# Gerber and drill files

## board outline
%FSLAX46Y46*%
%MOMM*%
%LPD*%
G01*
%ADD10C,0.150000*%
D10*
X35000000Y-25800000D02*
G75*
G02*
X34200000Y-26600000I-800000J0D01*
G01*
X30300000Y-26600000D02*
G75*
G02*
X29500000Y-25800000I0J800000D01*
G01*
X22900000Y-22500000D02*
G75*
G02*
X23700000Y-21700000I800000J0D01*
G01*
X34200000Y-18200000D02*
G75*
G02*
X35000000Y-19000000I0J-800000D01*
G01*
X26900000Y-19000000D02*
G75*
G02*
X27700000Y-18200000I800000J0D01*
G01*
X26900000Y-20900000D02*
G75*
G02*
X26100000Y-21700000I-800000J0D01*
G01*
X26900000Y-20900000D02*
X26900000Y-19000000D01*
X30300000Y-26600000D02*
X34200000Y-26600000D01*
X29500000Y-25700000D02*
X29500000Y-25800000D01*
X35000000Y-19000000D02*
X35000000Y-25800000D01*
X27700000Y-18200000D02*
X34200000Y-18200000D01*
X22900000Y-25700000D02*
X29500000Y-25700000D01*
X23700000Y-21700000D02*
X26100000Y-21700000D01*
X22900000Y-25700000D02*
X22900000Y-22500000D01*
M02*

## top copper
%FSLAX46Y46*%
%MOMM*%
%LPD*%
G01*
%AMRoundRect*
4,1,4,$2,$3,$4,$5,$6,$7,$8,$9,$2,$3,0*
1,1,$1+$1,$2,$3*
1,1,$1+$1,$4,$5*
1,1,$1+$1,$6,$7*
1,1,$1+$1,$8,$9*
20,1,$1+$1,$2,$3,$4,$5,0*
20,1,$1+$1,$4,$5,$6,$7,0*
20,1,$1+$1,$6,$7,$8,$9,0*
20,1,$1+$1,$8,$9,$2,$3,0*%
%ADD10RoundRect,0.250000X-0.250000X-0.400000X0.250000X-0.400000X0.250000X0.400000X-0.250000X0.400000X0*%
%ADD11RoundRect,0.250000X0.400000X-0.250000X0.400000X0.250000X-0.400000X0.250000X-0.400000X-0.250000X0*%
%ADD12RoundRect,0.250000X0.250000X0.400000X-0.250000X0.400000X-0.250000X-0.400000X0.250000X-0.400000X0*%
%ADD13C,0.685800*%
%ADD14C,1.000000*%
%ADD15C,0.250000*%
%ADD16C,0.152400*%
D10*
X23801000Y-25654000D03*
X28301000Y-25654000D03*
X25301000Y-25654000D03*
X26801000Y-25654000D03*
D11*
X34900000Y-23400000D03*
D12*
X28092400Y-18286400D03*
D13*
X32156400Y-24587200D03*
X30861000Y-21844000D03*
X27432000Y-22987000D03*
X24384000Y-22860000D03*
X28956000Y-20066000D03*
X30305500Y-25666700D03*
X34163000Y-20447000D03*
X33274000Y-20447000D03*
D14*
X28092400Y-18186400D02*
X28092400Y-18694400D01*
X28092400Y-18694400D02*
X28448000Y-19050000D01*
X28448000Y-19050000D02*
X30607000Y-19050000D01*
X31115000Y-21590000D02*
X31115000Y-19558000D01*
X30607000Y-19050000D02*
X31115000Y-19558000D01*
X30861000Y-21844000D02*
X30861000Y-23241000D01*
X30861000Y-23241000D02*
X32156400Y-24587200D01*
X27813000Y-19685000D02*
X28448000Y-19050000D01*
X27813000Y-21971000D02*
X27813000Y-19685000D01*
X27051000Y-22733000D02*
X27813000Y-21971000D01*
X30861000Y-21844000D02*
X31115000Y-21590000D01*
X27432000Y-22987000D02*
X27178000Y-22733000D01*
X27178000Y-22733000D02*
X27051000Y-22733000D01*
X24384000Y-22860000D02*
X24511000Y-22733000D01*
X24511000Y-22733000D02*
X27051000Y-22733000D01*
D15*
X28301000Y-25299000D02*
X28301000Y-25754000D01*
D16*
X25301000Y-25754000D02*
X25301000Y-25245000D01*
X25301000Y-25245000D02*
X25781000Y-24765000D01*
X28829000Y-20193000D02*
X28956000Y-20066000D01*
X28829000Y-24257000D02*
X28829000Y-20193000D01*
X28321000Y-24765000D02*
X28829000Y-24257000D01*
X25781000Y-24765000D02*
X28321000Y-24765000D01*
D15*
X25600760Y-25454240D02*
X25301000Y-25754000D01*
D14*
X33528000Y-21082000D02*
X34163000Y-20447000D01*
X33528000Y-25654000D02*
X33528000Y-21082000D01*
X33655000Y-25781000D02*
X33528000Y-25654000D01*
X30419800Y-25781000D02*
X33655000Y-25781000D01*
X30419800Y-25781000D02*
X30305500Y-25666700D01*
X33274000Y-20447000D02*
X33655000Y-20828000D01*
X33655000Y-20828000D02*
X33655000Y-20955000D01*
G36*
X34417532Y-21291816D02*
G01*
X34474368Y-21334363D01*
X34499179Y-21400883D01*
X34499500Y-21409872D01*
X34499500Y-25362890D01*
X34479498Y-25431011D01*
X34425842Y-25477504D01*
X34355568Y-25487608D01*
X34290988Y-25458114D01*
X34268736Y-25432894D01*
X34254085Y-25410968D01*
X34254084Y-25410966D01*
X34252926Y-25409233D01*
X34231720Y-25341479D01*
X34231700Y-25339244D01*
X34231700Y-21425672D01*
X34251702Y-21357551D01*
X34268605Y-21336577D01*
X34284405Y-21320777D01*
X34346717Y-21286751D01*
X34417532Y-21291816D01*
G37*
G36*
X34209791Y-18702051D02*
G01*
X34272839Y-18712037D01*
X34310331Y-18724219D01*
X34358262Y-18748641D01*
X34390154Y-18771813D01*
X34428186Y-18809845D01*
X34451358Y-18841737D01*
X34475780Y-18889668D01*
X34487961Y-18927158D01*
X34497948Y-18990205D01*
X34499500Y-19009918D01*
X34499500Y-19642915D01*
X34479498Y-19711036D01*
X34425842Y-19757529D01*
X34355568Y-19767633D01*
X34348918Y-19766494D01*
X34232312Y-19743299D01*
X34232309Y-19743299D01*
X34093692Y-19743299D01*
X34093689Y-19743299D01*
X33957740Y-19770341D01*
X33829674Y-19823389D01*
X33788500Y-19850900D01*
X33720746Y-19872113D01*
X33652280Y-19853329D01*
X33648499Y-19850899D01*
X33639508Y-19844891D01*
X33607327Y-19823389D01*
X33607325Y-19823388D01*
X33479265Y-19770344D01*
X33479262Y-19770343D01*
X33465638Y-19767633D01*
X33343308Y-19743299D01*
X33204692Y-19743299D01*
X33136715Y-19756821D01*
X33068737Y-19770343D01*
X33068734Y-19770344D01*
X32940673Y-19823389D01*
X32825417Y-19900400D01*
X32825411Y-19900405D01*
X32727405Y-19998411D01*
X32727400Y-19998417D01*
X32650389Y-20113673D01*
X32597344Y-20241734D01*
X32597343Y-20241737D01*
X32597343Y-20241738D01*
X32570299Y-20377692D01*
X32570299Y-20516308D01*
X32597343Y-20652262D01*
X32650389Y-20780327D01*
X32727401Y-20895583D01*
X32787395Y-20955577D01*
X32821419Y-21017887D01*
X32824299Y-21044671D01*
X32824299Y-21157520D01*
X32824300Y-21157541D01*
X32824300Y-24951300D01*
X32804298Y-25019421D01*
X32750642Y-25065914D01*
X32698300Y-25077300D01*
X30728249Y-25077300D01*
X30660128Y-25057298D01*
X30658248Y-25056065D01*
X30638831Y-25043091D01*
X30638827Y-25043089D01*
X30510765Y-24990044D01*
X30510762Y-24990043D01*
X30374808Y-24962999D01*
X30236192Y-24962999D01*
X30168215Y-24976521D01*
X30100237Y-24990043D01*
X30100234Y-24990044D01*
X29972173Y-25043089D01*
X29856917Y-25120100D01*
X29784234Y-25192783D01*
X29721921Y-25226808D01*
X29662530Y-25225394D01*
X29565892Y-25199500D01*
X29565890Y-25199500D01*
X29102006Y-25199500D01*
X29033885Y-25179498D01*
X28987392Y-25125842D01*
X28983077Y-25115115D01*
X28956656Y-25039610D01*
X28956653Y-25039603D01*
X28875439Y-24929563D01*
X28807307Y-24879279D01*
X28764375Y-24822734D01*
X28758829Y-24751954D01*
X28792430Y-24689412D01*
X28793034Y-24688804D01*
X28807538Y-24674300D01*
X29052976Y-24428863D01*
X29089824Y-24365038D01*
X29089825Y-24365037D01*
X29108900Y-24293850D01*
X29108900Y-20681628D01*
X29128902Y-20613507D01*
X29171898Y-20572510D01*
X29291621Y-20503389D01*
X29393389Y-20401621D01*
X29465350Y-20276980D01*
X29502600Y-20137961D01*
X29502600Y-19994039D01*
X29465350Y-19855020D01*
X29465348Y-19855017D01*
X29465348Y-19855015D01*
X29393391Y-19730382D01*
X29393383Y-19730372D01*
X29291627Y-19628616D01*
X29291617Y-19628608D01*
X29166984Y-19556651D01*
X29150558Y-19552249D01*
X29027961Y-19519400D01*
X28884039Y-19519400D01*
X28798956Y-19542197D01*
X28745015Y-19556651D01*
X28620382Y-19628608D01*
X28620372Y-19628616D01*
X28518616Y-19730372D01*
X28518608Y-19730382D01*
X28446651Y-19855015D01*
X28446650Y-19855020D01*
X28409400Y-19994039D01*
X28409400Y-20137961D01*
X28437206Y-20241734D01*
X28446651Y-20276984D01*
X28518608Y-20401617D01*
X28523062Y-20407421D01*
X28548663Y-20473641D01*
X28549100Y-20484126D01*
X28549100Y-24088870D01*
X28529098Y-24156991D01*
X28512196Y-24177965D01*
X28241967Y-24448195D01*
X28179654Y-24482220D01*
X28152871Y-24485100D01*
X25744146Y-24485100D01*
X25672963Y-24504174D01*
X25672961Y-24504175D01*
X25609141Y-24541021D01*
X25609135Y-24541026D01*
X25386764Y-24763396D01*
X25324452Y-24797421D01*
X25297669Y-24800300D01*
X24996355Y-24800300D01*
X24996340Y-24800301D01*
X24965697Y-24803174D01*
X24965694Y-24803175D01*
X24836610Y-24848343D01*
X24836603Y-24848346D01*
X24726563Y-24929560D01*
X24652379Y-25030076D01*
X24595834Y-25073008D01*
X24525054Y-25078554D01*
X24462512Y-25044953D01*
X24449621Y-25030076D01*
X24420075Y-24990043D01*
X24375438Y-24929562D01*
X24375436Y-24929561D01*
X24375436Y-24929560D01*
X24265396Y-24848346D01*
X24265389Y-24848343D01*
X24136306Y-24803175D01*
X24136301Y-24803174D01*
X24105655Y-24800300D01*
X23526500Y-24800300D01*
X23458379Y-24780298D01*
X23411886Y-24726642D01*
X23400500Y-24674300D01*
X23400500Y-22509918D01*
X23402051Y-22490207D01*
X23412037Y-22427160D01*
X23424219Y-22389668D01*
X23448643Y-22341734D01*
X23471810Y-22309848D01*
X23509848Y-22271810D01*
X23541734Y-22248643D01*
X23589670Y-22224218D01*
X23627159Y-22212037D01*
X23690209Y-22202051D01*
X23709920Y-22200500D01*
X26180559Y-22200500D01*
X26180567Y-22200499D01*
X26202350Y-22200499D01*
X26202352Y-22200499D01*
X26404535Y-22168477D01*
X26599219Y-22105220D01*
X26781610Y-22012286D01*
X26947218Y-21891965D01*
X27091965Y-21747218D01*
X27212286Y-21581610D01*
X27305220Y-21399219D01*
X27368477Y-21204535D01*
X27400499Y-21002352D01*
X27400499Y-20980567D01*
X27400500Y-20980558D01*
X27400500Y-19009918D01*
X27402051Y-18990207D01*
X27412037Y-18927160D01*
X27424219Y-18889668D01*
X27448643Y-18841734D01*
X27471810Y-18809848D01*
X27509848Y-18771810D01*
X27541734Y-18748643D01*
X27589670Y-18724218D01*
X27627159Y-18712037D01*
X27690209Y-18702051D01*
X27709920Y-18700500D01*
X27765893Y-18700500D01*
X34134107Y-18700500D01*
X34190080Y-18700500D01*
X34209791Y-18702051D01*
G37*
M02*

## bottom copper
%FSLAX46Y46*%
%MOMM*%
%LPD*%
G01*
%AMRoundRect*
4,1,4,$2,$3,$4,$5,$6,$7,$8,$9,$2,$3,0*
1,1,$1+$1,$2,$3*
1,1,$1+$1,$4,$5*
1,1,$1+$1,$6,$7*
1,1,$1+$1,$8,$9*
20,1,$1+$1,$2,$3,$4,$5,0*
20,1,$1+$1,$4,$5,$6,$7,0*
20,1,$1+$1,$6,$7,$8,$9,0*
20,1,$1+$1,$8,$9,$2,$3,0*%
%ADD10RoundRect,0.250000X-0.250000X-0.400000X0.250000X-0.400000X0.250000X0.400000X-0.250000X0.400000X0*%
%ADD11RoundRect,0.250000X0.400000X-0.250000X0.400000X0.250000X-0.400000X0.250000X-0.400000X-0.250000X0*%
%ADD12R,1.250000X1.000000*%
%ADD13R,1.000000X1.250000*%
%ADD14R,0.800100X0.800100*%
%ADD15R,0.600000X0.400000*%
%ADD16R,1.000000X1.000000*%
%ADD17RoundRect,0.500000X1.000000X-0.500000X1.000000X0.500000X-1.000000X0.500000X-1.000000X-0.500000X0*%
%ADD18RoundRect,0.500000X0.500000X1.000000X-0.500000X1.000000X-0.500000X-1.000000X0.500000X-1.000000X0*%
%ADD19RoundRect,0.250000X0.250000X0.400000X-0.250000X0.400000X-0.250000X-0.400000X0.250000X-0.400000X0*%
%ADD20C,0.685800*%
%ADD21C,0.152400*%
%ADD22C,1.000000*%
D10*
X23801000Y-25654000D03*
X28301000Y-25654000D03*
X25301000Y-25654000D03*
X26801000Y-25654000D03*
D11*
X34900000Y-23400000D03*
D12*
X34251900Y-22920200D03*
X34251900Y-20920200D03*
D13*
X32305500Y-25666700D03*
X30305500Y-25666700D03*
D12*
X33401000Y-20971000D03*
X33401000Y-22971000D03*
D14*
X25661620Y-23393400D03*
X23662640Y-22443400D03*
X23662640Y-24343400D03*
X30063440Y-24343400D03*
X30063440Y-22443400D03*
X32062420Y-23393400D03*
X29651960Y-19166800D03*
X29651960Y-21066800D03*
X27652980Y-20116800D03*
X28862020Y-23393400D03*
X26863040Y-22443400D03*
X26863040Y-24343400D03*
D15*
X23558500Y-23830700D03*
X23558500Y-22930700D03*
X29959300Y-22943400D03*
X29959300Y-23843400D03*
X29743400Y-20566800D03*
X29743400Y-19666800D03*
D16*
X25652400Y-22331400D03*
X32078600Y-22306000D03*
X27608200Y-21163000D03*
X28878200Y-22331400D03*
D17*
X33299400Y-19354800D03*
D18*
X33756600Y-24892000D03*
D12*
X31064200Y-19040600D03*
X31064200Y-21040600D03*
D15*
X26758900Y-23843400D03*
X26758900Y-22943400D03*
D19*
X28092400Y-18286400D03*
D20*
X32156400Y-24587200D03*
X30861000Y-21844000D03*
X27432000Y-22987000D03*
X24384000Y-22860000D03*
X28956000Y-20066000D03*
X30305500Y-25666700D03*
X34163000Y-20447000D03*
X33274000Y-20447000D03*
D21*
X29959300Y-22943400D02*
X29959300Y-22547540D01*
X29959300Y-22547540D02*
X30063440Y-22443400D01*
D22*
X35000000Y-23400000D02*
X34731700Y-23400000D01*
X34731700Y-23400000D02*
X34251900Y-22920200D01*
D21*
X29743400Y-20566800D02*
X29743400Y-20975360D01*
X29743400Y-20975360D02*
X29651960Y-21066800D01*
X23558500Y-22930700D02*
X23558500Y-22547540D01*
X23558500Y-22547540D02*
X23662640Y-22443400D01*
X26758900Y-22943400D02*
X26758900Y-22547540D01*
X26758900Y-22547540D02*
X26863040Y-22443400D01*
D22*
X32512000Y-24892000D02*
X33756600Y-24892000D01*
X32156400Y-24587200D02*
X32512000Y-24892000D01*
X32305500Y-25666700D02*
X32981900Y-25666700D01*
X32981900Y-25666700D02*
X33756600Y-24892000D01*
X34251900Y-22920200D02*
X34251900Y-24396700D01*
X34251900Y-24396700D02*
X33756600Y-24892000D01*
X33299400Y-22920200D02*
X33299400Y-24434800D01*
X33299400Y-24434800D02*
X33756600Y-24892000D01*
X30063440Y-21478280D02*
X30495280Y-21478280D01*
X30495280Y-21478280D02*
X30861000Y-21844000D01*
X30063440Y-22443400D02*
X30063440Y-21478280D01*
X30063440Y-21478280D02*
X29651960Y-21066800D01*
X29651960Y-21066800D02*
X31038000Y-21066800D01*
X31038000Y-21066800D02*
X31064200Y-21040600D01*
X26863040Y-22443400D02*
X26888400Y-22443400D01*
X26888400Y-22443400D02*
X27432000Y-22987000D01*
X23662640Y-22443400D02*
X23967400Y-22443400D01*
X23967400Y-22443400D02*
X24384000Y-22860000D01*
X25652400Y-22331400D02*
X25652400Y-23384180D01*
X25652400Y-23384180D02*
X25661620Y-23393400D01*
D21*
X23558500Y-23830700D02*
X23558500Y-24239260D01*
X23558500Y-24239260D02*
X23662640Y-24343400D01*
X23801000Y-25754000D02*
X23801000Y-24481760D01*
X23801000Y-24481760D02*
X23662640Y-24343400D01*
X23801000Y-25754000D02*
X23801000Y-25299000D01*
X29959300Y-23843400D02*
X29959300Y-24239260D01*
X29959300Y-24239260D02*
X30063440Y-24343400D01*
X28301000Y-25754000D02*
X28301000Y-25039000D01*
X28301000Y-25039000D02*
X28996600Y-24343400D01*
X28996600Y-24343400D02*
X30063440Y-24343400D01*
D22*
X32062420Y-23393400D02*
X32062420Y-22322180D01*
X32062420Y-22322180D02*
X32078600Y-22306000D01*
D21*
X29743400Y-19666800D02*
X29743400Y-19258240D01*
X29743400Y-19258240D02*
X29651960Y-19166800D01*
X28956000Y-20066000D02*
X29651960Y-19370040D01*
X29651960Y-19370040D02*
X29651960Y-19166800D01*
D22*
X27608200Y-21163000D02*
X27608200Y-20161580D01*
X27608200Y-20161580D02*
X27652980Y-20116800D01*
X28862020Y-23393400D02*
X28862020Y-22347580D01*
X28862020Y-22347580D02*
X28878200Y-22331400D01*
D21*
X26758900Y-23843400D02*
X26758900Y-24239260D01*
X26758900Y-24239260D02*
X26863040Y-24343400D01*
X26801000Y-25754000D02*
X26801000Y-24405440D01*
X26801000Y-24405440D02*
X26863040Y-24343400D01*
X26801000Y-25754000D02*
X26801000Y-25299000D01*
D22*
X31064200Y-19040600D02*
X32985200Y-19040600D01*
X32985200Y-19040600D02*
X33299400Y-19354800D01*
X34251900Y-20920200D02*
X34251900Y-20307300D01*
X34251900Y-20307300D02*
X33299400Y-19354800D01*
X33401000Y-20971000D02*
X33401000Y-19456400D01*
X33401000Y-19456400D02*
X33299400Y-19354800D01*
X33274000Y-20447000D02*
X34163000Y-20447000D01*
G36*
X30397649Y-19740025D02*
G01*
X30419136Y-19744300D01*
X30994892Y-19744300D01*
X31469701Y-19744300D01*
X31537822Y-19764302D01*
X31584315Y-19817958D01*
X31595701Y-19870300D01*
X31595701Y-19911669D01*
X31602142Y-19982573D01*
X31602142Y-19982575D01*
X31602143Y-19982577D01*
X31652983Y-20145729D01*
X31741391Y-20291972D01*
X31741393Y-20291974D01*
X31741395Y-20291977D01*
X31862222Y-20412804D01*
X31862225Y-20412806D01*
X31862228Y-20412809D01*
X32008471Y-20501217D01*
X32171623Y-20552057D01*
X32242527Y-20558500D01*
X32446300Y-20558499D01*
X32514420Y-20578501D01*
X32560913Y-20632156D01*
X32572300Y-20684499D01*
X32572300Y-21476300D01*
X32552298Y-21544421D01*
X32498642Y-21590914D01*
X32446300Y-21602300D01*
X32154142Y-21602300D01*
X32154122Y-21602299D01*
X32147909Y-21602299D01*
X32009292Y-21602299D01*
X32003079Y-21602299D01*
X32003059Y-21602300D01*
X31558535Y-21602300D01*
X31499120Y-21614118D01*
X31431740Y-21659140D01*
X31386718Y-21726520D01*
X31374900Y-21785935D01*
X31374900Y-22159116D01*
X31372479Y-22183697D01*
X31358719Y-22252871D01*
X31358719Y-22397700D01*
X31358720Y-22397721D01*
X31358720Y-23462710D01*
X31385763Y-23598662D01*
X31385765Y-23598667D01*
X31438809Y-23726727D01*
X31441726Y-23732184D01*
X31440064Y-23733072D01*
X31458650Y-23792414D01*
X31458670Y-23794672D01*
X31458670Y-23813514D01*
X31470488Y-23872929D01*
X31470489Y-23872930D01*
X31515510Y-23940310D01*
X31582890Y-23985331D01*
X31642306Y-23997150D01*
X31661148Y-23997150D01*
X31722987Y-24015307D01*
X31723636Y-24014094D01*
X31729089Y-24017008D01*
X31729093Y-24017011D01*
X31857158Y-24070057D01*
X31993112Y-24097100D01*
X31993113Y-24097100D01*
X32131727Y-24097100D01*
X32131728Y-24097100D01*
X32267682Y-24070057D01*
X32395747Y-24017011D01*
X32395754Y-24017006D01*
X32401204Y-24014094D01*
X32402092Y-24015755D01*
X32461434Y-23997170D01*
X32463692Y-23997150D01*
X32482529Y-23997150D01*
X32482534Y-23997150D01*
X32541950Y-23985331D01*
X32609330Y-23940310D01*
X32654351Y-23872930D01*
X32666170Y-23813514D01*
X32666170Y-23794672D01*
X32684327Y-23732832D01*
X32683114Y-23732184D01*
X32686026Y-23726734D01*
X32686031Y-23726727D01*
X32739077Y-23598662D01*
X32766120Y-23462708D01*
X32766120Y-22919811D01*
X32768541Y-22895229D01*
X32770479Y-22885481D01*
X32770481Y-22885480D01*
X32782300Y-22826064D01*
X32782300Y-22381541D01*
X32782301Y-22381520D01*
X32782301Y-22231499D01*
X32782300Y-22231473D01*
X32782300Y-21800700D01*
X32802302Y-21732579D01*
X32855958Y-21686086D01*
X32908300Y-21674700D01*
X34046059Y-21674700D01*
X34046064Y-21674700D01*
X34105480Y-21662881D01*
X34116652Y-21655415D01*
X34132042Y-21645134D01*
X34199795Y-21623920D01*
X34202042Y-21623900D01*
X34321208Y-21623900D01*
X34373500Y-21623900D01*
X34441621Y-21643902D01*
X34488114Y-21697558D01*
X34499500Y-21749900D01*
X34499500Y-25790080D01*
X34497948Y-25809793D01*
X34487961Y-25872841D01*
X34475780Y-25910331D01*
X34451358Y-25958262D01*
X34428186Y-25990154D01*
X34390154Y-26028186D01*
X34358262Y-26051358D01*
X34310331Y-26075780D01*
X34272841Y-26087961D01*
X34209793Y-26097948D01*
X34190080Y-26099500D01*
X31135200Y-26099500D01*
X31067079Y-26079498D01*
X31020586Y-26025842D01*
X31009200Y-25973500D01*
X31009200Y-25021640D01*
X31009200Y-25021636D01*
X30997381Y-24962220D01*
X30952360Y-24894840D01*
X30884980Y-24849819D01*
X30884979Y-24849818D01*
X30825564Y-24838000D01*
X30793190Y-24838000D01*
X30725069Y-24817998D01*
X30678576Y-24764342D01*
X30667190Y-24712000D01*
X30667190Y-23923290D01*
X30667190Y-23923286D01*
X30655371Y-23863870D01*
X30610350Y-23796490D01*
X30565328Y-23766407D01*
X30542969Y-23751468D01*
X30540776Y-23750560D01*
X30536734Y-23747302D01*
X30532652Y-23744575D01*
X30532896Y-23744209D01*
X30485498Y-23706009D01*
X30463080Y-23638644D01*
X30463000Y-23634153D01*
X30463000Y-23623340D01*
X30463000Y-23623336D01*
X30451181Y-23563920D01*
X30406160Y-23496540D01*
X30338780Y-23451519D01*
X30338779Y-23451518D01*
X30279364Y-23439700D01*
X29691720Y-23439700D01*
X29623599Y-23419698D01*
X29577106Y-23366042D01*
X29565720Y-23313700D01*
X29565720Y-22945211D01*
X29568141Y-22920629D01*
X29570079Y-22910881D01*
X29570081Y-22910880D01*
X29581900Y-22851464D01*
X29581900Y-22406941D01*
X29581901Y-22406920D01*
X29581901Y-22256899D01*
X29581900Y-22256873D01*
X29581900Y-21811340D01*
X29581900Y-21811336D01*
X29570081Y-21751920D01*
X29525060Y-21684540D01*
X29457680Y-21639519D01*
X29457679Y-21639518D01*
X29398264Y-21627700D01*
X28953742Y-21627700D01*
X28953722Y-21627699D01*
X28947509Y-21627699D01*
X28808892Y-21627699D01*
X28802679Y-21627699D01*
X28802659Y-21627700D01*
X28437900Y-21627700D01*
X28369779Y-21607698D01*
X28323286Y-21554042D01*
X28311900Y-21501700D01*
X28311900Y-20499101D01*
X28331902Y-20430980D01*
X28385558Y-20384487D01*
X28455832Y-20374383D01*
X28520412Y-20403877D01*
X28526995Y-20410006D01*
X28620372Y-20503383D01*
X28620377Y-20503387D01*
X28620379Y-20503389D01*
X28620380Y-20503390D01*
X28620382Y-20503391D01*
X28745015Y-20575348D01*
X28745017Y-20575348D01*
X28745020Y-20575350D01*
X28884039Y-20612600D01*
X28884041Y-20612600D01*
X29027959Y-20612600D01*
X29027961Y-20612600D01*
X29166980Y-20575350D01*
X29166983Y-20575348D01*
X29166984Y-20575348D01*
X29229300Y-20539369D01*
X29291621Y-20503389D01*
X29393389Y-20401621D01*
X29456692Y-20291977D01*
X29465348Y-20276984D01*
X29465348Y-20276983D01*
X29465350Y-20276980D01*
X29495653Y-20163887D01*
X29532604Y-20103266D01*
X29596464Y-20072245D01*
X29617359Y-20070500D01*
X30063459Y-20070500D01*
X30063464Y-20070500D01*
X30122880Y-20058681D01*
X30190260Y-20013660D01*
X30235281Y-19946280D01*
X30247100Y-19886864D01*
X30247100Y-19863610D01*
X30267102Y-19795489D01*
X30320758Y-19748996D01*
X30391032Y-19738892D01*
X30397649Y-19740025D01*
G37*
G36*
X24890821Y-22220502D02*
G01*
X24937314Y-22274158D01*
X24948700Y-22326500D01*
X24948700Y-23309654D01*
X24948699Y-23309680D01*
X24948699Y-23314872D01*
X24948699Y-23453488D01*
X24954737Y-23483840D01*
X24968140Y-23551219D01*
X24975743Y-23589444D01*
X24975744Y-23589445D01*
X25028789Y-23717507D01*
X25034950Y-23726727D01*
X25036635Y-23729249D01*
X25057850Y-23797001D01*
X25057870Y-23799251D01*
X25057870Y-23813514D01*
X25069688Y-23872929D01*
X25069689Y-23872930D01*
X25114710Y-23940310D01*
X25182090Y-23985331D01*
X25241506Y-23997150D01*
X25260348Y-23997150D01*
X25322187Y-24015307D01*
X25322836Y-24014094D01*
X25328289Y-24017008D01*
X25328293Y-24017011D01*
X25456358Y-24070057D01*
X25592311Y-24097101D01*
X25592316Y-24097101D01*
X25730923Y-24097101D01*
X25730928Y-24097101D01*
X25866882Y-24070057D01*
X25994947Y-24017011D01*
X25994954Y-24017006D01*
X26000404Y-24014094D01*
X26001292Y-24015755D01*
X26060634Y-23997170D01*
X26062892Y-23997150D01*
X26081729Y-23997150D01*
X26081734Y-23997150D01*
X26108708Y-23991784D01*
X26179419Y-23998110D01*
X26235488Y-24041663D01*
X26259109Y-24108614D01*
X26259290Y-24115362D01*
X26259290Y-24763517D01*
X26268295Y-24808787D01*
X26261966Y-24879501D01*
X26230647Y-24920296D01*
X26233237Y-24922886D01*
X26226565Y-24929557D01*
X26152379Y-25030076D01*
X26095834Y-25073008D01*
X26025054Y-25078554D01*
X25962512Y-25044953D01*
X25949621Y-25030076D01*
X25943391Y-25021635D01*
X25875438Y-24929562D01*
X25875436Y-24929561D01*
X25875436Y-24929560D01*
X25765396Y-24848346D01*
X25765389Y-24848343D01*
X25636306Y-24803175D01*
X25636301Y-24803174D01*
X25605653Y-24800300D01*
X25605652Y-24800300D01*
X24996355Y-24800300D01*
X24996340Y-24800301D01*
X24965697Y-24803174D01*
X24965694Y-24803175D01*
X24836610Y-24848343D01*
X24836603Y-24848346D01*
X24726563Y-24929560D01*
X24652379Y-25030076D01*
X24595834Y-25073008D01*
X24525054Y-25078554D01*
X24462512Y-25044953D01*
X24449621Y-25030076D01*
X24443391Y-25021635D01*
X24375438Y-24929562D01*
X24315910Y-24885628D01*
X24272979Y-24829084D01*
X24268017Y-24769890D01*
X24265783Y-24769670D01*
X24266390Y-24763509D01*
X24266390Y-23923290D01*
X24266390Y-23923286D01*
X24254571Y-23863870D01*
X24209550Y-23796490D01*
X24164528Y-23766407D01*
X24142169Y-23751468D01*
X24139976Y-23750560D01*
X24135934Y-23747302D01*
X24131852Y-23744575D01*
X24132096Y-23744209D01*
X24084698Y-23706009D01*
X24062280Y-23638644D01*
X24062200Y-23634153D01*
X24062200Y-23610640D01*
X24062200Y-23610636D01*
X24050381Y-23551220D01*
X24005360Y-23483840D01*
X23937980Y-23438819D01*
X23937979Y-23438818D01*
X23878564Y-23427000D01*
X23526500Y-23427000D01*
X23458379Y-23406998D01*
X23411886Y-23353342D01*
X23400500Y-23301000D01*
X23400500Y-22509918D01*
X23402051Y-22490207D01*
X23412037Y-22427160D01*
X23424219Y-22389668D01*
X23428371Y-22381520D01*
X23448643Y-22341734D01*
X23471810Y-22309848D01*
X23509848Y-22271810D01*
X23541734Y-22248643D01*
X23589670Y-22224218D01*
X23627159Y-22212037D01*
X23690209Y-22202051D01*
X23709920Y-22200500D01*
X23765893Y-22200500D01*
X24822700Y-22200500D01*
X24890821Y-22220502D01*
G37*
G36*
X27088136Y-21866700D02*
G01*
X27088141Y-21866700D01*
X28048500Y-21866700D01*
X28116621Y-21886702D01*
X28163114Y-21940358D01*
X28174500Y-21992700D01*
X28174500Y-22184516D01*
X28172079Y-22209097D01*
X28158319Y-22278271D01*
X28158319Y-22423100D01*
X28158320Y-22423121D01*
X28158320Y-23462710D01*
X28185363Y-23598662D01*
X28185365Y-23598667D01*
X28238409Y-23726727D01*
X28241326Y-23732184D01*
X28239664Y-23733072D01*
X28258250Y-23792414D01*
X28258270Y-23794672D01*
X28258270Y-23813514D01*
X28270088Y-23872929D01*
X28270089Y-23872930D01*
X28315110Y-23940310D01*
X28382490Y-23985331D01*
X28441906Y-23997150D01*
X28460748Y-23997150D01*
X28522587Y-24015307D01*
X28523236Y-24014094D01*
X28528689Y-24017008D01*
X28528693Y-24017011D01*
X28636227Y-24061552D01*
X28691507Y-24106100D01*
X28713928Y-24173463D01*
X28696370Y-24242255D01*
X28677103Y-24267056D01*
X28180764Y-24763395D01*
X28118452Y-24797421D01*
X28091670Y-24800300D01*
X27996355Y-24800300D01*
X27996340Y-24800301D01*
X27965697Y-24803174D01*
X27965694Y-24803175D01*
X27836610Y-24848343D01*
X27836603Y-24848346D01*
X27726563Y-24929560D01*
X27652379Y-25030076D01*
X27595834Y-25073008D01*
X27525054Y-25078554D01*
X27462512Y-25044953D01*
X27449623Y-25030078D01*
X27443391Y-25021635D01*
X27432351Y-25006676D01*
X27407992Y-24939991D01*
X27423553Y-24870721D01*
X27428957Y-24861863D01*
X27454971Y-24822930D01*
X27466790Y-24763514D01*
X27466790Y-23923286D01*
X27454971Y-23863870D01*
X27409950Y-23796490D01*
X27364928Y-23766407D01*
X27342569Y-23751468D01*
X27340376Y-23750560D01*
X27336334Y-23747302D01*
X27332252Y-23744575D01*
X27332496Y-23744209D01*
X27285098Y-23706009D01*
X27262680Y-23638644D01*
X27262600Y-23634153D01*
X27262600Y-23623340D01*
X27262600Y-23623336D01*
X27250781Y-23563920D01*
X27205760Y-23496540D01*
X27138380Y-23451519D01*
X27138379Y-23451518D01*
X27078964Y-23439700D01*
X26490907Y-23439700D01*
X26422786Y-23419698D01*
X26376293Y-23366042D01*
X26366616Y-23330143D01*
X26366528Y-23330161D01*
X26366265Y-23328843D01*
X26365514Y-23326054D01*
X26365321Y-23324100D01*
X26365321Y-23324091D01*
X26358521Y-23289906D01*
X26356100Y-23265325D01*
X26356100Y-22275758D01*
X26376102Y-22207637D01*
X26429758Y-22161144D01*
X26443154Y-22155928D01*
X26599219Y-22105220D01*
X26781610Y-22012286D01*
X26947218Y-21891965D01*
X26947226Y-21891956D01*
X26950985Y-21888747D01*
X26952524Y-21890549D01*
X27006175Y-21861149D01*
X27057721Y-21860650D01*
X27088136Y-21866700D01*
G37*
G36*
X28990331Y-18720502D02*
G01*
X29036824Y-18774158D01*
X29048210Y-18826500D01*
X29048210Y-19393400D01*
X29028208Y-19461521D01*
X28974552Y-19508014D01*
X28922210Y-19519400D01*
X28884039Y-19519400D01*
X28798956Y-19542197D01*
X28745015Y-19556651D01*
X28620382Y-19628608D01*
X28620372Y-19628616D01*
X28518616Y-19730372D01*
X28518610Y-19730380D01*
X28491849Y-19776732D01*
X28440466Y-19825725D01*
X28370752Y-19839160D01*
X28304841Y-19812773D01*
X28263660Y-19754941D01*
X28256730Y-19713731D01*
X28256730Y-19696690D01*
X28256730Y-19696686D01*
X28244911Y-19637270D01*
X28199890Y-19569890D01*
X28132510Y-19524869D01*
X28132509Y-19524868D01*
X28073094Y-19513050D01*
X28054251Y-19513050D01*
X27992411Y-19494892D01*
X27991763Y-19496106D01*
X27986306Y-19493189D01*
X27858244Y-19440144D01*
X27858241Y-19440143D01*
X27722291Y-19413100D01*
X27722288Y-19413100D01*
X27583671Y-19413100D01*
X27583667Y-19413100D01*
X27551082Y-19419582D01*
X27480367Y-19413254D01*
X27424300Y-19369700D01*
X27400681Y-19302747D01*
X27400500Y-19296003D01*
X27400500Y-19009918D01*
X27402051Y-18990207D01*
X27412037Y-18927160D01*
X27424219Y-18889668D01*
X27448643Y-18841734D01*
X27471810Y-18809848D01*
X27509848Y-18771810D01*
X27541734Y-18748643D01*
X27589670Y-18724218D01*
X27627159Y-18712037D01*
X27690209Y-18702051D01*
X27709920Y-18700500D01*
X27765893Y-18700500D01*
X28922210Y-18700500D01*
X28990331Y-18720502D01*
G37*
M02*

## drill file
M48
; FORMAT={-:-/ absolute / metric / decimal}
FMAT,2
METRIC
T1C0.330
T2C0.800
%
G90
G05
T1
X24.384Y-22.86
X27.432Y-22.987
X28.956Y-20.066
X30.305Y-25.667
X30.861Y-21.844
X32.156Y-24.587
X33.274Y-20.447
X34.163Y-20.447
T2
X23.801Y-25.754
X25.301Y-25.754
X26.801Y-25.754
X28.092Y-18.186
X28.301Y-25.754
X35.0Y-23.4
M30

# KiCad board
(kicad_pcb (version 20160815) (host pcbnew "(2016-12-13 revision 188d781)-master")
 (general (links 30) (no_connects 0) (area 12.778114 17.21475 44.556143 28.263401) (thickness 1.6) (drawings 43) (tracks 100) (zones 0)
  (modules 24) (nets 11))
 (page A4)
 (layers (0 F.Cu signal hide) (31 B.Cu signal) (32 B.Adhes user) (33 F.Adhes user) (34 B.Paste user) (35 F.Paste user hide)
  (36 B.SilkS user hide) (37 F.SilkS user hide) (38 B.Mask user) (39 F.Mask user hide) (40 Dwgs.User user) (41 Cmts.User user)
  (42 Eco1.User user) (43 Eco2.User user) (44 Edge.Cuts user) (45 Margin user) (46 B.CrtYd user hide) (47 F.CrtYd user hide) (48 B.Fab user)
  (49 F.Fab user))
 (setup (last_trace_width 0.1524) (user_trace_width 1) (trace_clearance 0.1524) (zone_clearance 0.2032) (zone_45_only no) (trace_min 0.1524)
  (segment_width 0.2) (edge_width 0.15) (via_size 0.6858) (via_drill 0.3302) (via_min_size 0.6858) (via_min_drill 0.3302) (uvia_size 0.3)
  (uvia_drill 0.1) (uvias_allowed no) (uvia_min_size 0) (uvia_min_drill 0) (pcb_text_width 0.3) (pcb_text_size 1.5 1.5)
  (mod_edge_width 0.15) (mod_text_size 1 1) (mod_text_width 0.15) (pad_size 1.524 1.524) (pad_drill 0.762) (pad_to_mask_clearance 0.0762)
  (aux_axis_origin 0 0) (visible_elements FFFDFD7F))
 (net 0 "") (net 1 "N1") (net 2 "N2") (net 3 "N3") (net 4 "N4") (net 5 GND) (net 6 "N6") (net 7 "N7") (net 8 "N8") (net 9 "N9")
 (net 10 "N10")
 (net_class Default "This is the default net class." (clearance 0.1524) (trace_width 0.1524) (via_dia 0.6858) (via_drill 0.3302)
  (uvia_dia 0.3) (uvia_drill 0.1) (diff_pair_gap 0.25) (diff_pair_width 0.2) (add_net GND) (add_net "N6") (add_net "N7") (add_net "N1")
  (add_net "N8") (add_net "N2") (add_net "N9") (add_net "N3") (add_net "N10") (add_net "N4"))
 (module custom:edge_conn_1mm (layer F.Cu) (at 23.801 25.754)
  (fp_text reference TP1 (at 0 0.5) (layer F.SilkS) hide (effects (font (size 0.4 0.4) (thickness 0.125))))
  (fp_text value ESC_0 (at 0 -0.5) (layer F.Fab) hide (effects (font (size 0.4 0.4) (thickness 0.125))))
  (pad 1 thru_hole roundrect (at 0 0) (size 1 1.3) (drill 0.8 (offset 0 -0.1)) (layers *.Cu *.Mask) (roundrect_rratio 0.25) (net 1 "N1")))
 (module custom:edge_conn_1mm (layer F.Cu) (at 28.301 25.754)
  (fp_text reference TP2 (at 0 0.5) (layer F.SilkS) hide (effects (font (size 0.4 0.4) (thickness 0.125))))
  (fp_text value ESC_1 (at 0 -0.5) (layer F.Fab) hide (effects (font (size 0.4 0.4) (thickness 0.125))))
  (pad 1 thru_hole roundrect (at 0 0) (size 1 1.3) (drill 0.8 (offset 0 -0.1)) (layers *.Cu *.Mask) (roundrect_rratio 0.25) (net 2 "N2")))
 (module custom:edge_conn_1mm (layer F.Cu) (at 25.301 25.754)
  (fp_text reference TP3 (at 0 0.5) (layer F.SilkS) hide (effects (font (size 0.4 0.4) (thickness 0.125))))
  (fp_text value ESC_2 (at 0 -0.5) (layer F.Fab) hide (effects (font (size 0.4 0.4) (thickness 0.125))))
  (pad 1 thru_hole roundrect (at 0 0) (size 1 1.3) (drill 0.8 (offset 0 -0.1)) (layers *.Cu *.Mask) (roundrect_rratio 0.25) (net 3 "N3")))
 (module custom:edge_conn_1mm (layer F.Cu) (at 26.801 25.754)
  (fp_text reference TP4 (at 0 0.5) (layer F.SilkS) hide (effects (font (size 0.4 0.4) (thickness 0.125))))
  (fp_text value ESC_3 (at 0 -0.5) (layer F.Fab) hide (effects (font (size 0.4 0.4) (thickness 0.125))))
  (pad 1 thru_hole roundrect (at 0 0) (size 1 1.3) (drill 0.8 (offset 0 -0.1)) (layers *.Cu *.Mask) (roundrect_rratio 0.25) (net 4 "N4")))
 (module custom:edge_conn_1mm (layer F.Cu) (at 35 23.4 90)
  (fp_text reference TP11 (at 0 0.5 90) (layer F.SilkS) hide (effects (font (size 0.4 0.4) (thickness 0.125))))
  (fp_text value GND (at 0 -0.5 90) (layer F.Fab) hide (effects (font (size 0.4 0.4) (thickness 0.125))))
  (pad 1 thru_hole roundrect (at 0 0 90) (size 1 1.3) (drill 0.8 (offset 0 -0.1)) (layers *.Cu *.Mask) (roundrect_rratio 0.25) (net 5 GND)))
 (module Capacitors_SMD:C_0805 (layer B.Cu) (at 34.2519 21.9202 270)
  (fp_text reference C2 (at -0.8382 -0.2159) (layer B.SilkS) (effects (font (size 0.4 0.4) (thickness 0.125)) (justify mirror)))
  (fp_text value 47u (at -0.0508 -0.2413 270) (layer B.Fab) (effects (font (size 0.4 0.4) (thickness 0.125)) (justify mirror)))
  (pad 2 smd rect (at 1 0 270) (size 1 1.25) (layers B.Cu B.Paste B.Mask) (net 5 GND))
  (pad 1 smd rect (at -1 0 270) (size 1 1.25) (layers B.Cu B.Paste B.Mask) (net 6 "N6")))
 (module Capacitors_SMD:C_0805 (layer B.Cu) (at 31.3055 25.6667)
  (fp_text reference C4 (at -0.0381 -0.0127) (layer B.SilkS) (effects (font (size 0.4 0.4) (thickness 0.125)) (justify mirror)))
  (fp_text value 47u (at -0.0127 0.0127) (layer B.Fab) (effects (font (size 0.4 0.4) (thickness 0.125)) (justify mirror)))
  (pad 2 smd rect (at 1 0) (size 1 1.25) (layers B.Cu B.Paste B.Mask) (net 5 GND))
  (pad 1 smd rect (at -1 0) (size 1 1.25) (layers B.Cu B.Paste B.Mask) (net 6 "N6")))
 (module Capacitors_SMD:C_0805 (layer B.Cu) (at 33.401 21.971 270)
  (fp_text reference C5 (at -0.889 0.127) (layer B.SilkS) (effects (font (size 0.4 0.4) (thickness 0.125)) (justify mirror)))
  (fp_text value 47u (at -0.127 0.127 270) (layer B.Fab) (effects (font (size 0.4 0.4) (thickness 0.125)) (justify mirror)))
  (pad 1 smd rect (at -1 0 270) (size 1 1.25) (layers B.Cu B.Paste B.Mask) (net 6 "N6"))
  (pad 2 smd rect (at 1 0 270) (size 1 1.25) (layers B.Cu B.Paste B.Mask) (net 5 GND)))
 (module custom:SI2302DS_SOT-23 (layer B.Cu) (at 24.6634 23.3934 90)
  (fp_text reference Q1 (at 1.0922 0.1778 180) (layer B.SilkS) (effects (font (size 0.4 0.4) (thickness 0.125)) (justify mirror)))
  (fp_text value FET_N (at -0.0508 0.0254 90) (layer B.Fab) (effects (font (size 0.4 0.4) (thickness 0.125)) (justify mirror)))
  (pad D smd rect (at 0 0.99822 90) (size 0.8001 0.8001) (layers B.Cu B.Paste B.Mask) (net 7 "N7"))
  (pad S smd rect (at 0.95 -1.00076 90) (size 0.8001 0.8001) (layers B.Cu B.Paste B.Mask) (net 5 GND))
  (pad G smd rect (at -0.95 -1.00076 90) (size 0.8001 0.8001) (layers B.Cu B.Paste B.Mask) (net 1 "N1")))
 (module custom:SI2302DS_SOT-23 (layer B.Cu) (at 31.0642 23.3934 90)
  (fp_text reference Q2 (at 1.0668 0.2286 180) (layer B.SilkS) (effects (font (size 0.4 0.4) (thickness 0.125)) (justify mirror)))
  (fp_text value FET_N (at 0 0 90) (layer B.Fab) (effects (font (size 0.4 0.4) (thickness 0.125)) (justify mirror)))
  (pad G smd rect (at -0.95 -1.00076 90) (size 0.8001 0.8001) (layers B.Cu B.Paste B.Mask) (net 2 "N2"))
  (pad S smd rect (at 0.95 -1.00076 90) (size 0.8001 0.8001) (layers B.Cu B.Paste B.Mask) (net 5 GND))
  (pad D smd rect (at 0 0.99822 90) (size 0.8001 0.8001) (layers B.Cu B.Paste B.Mask) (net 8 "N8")))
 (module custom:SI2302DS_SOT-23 (layer B.Cu) (at 28.6512 20.1168 270)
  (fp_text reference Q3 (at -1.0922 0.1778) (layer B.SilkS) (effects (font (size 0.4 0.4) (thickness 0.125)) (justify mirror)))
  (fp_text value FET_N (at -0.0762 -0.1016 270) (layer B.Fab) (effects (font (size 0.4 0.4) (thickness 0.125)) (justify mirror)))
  (pad G smd rect (at -0.95 -1.00076 270) (size 0.8001 0.8001) (layers B.Cu B.Paste B.Mask) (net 3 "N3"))
  (pad S smd rect (at 0.95 -1.00076 270) (size 0.8001 0.8001) (layers B.Cu B.Paste B.Mask) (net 5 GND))
  (pad D smd rect (at 0 0.99822 270) (size 0.8001 0.8001) (layers B.Cu B.Paste B.Mask) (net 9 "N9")))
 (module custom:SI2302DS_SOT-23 (layer B.Cu) (at 27.8638 23.3934 90)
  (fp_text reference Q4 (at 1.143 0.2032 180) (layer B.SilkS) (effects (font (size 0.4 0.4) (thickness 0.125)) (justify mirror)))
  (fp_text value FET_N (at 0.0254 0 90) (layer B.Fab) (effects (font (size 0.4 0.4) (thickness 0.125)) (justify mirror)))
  (pad D smd rect (at 0 0.99822 90) (size 0.8001 0.8001) (layers B.Cu B.Paste B.Mask) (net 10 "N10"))
  (pad S smd rect (at 0.95 -1.00076 90) (size 0.8001 0.8001) (layers B.Cu B.Paste B.Mask) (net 5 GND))
  (pad G smd rect (at -0.95 -1.00076 90) (size 0.8001 0.8001) (layers B.Cu B.Paste B.Mask) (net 4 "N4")))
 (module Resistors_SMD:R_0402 (layer B.Cu) (at 23.5585 23.3807 90)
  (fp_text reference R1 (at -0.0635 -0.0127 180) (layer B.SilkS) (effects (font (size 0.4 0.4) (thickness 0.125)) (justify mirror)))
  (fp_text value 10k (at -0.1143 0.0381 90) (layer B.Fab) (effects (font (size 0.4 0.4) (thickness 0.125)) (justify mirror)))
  (pad 1 smd rect (at -0.45 0 90) (size 0.4 0.6) (layers B.Cu B.Paste B.Mask) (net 1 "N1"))
  (pad 2 smd rect (at 0.45 0 90) (size 0.4 0.6) (layers B.Cu B.Paste B.Mask) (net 5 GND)))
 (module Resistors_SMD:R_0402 (layer B.Cu) (at 29.9593 23.3934 90)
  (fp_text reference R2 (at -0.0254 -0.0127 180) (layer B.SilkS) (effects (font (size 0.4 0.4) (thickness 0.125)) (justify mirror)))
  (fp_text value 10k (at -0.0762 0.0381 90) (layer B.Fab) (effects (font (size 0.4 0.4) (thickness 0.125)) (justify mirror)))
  (pad 2 smd rect (at 0.45 0 90) (size 0.4 0.6) (layers B.Cu B.Paste B.Mask) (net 5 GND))
  (pad 1 smd rect (at -0.45 0 90) (size 0.4 0.6) (layers B.Cu B.Paste B.Mask) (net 2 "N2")))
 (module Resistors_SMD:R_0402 (layer B.Cu) (at 29.7434 20.1168 270)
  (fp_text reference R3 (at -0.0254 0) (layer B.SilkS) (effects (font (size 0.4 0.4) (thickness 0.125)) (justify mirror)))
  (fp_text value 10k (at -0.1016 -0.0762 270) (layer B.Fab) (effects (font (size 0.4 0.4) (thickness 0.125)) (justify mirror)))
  (pad 2 smd rect (at 0.45 0 270) (size 0.4 0.6) (layers B.Cu B.Paste B.Mask) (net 5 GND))
  (pad 1 smd rect (at -0.45 0 270) (size 0.4 0.6) (layers B.Cu B.Paste B.Mask) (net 3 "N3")))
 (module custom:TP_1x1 (layer B.Cu) (at 25.5524 22.6314)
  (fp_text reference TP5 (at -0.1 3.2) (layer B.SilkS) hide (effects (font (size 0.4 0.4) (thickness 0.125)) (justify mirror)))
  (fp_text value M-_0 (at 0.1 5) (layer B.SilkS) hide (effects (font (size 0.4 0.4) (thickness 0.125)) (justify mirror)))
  (pad 1 smd rect (at 0.1 -0.3) (size 1 1) (layers B.Cu B.Mask) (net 7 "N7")))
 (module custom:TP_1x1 (layer B.Cu) (at 31.9786 22.606)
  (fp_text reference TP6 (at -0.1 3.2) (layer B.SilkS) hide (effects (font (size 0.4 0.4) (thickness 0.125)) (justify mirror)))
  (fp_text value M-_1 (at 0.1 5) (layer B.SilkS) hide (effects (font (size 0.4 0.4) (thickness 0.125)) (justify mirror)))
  (pad 1 smd rect (at 0.1 -0.3) (size 1 1) (layers B.Cu B.Mask) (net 8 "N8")))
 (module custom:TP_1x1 (layer B.Cu) (at 27.5082 21.463)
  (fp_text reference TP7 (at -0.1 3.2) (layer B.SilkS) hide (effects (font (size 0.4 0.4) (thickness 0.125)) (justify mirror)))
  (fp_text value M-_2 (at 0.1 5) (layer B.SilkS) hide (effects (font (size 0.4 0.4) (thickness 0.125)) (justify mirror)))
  (pad 1 smd rect (at 0.1 -0.3) (size 1 1) (layers B.Cu B.Mask) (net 9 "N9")))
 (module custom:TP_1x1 (layer B.Cu) (at 28.7782 22.6314)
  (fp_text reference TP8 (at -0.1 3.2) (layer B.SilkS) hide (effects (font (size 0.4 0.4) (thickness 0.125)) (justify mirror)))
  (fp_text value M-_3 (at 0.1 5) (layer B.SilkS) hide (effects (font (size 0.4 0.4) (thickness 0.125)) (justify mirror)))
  (pad 1 smd rect (at 0.1 -0.3) (size 1 1) (layers B.Cu B.Mask) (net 10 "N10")))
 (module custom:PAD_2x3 (layer B.Cu) (at 33.2994 19.3548 90)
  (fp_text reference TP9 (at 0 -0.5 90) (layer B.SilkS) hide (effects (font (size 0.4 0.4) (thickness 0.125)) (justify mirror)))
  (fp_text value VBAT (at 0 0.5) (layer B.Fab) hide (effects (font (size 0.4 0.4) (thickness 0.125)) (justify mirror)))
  (pad 1 smd roundrect (at 0 0 90) (size 2 3) (layers B.Cu B.Mask) (roundrect_rratio 0.25) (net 6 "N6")))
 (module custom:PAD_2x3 (layer B.Cu) (at 33.7566 24.892 180)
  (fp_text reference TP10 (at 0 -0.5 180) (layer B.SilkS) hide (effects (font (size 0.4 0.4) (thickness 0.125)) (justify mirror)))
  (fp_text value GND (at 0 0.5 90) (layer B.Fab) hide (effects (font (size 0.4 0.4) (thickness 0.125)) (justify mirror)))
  (pad 1 smd roundrect (at 0 0 180) (size 2 3) (layers B.Cu B.Mask) (roundrect_rratio 0.25) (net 5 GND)))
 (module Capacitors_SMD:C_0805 (layer B.Cu) (at 31.0642 20.0406 270)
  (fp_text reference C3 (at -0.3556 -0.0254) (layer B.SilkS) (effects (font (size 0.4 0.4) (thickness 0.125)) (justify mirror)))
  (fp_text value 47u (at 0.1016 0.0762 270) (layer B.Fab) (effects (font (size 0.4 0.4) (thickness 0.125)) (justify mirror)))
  (pad 1 smd rect (at -1 0 270) (size 1 1.25) (layers B.Cu B.Paste B.Mask) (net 6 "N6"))
  (pad 2 smd rect (at 1 0 270) (size 1 1.25) (layers B.Cu B.Paste B.Mask) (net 5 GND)))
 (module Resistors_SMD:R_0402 (layer B.Cu) (at 26.7589 23.3934 90)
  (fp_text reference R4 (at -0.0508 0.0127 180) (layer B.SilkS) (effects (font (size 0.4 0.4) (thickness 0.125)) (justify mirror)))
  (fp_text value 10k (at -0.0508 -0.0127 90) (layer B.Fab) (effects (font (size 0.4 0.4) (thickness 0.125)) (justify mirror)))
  (pad 1 smd rect (at -0.45 0 90) (size 0.4 0.6) (layers B.Cu B.Paste B.Mask) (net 4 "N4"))
  (pad 2 smd rect (at 0.45 0 90) (size 0.4 0.6) (layers B.Cu B.Paste B.Mask) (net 5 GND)))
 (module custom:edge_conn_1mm (layer F.Cu) (at 28.0924 18.1864 180)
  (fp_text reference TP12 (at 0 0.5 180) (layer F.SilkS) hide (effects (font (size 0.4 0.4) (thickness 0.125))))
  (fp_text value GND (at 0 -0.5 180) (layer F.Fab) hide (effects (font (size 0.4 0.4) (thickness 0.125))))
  (pad 1 thru_hole roundrect (at 0 0 180) (size 1 1.3) (drill 0.8 (offset 0 -0.1)) (layers *.Cu *.Mask) (roundrect_rratio 0.25) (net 5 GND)))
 (gr_arc (start 34.2 25.8) (end 35 25.8) (angle 90) (layer Edge.Cuts) (width 0.15))
 (gr_arc (start 30.3 25.8) (end 30.3 26.6) (angle 90) (layer Edge.Cuts) (width 0.15))
 (gr_arc (start 23.7 22.5) (end 22.9 22.5) (angle 90) (layer Edge.Cuts) (width 0.15))
 (gr_arc (start 34.2 19) (end 34.2 18.2) (angle 90) (layer Edge.Cuts) (width 0.15))
 (gr_arc (start 27.7 19) (end 26.9 19) (angle 90) (layer Edge.Cuts) (width 0.15))
 (gr_arc (start 26.1 20.9) (end 26.9 20.9) (angle 90) (layer Edge.Cuts) (width 0.15))
 (gr_line (start 26.9 20.9) (end 26.9 19) (angle 90) (layer Edge.Cuts) (width 0.15))
 (gr_line (start 30.3 26.6) (end 34.2 26.6) (angle 90) (layer Edge.Cuts) (width 0.15))
 (gr_line (start 29.5 25.7) (end 29.5 25.8) (angle 90) (layer Edge.Cuts) (width 0.15))
 (gr_line (start 35 19) (end 35 25.8) (angle 90) (layer Edge.Cuts) (width 0.15))
 (gr_line (start 27.7 18.2) (end 34.2 18.2) (angle 90) (layer Edge.Cuts) (width 0.15))
 (gr_line (start 22.9 25.7) (end 29.5 25.7) (angle 90) (layer Edge.Cuts) (width 0.15))
 (gr_line (start 23.7 21.7) (end 26.1 21.7) (angle 90) (layer Edge.Cuts) (width 0.15))
 (gr_line (start 22.9 25.7) (end 22.9 22.5) (angle 90) (layer Edge.Cuts) (width 0.15))
 (segment (start 28.0924 18.1864) (end 28.0924 18.6944) (width 1) (layer F.Cu) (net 5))
 (segment (start 28.0924 18.6944) (end 28.448 19.05) (width 1) (layer F.Cu) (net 5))
 (segment (start 29.9593 22.9434) (end 29.9593 22.54754) (width 0.1524) (layer B.Cu) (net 5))
 (segment (start 29.9593 22.54754) (end 30.06344 22.4434) (width 0.1524) (layer B.Cu) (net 5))
 (segment (start 35 23.4) (end 34.7317 23.4) (width 1) (layer B.Cu) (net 5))
 (segment (start 34.7317 23.4) (end 34.2519 22.9202) (width 1) (layer B.Cu) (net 5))
 (segment (start 28.448 19.05) (end 30.607 19.05) (width 1) (layer F.Cu) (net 5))
 (segment (start 31.115 21.59) (end 31.115 19.558) (width 1) (layer F.Cu) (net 5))
 (segment (start 30.607 19.05) (end 31.115 19.558) (width 1) (layer F.Cu) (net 5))
 (segment (start 29.7434 20.5668) (end 29.7434 20.97536) (width 0.1524) (layer B.Cu) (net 5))
 (segment (start 29.7434 20.97536) (end 29.65196 21.0668) (width 0.1524) (layer B.Cu) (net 5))
 (segment (start 23.5585 22.9307) (end 23.5585 22.54754) (width 0.1524) (layer B.Cu) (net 5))
 (segment (start 23.5585 22.54754) (end 23.66264 22.4434) (width 0.1524) (layer B.Cu) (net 5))
 (segment (start 26.7589 22.9434) (end 26.7589 22.54754) (width 0.1524) (layer B.Cu) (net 5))
 (segment (start 26.7589 22.54754) (end 26.86304 22.4434) (width 0.1524) (layer B.Cu) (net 5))
 (segment (start 30.861 21.844) (end 30.861 23.241) (width 1) (layer F.Cu) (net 5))
 (segment (start 32.512 24.892) (end 33.7566 24.892) (width 1) (layer B.Cu) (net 5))
 (segment (start 32.1564 24.5872) (end 32.512 24.892) (width 1) (layer B.Cu) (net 5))
 (via (at 32.1564 24.5872) (size 0.6858) (drill 0.3302) (layers F.Cu B.Cu) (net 5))
 (segment (start 30.861 23.241) (end 32.1564 24.5872) (width 1) (layer F.Cu) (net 5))
 (segment (start 32.3055 25.6667) (end 32.9819 25.6667) (width 1) (layer B.Cu) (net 5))
 (segment (start 32.9819 25.6667) (end 33.7566 24.892) (width 1) (layer B.Cu) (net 5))
 (segment (start 34.2519 22.9202) (end 34.2519 24.3967) (width 1) (layer B.Cu) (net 5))
 (segment (start 34.2519 24.3967) (end 33.7566 24.892) (width 1) (layer B.Cu) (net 5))
 (segment (start 33.2994 22.9202) (end 33.2994 24.4348) (width 1) (layer B.Cu) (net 5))
 (segment (start 33.2994 24.4348) (end 33.7566 24.892) (width 1) (layer B.Cu) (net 5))
 (segment (start 30.06344 21.47828) (end 30.49528 21.47828) (width 1) (layer B.Cu) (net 5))
 (segment (start 30.49528 21.47828) (end 30.861 21.844) (width 1) (layer B.Cu) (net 5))
 (segment (start 27.813 19.685) (end 28.448 19.05) (width 1) (layer F.Cu) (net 5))
 (segment (start 27.813 21.971) (end 27.813 19.685) (width 1) (layer F.Cu) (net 5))
 (segment (start 27.051 22.733) (end 27.813 21.971) (width 1) (layer F.Cu) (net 5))
 (segment (start 30.861 21.844) (end 31.115 21.59) (width 1) (layer F.Cu) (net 5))
 (via (at 30.861 21.844) (size 0.6858) (drill 0.3302) (layers F.Cu B.Cu) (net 5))
 (segment (start 30.06344 22.4434) (end 30.06344 21.47828) (width 1) (layer B.Cu) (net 5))
 (segment (start 30.06344 21.47828) (end 29.65196 21.0668) (width 1) (layer B.Cu) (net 5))
 (segment (start 29.65196 21.0668) (end 31.038 21.0668) (width 1) (layer B.Cu) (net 5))
 (segment (start 31.038 21.0668) (end 31.0642 21.0406) (width 1) (layer B.Cu) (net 5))
 (segment (start 26.86304 22.4434) (end 26.8884 22.4434) (width 1) (layer B.Cu) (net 5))
 (segment (start 26.8884 22.4434) (end 27.432 22.987) (width 1) (layer B.Cu) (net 5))
 (via (at 27.432 22.987) (size 0.6858) (drill 0.3302) (layers F.Cu B.Cu) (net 5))
 (segment (start 27.432 22.987) (end 27.178 22.733) (width 1) (layer F.Cu) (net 5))
 (segment (start 27.178 22.733) (end 27.051 22.733) (width 1) (layer F.Cu) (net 5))
 (segment (start 23.66264 22.4434) (end 23.9674 22.4434) (width 1) (layer B.Cu) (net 5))
 (segment (start 23.9674 22.4434) (end 24.384 22.86) (width 1) (layer B.Cu) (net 5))
 (via (at 24.384 22.86) (size 0.6858) (drill 0.3302) (layers F.Cu B.Cu) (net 5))
 (segment (start 24.384 22.86) (end 24.511 22.733) (width 1) (layer F.Cu) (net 5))
 (segment (start 24.511 22.733) (end 27.051 22.733) (width 1) (layer F.Cu) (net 5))
 (segment (start 25.6524 22.3314) (end 25.6524 23.38418) (width 1) (layer B.Cu) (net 7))
 (segment (start 25.6524 23.38418) (end 25.66162 23.3934) (width 1) (layer B.Cu) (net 7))
 (segment (start 23.5585 23.8307) (end 23.5585 24.23926) (width 0.1524) (layer B.Cu) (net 1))
 (segment (start 23.5585 24.23926) (end 23.66264 24.3434) (width 0.1524) (layer B.Cu) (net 1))
 (segment (start 23.801 25.754) (end 23.801 24.48176) (width 0.1524) (layer B.Cu) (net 1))
 (segment (start 23.801 24.48176) (end 23.66264 24.3434) (width 0.1524) (layer B.Cu) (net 1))
 (segment (start 23.801 25.754) (end 23.801 25.299) (width 0.1524) (layer B.Cu) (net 1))
 (segment (start 29.9593 23.8434) (end 29.9593 24.23926) (width 0.1524) (layer B.Cu) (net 2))
 (segment (start 29.9593 24.23926) (end 30.06344 24.3434) (width 0.1524) (layer B.Cu) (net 2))
 (segment (start 28.301 25.754) (end 28.301 25.039) (width 0.1524) (layer B.Cu) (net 2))
 (segment (start 28.301 25.039) (end 28.9966 24.3434) (width 0.1524) (layer B.Cu) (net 2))
 (segment (start 28.9966 24.3434) (end 30.06344 24.3434) (width 0.1524) (layer B.Cu) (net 2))
 (segment (start 28.301 25.299) (end 28.301 25.754) (width 0.25) (layer F.Cu) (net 2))
 (segment (start 32.06242 23.3934) (end 32.06242 22.32218) (width 1) (layer B.Cu) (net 8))
 (segment (start 32.06242 22.32218) (end 32.0786 22.306) (width 1) (layer B.Cu) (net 8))
 (segment (start 29.7434 19.6668) (end 29.7434 19.25824) (width 0.1524) (layer B.Cu) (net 3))
 (segment (start 29.7434 19.25824) (end 29.65196 19.1668) (width 0.1524) (layer B.Cu) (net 3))
 (segment (start 25.301 25.754) (end 25.301 25.245) (width 0.1524) (layer F.Cu) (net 3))
 (segment (start 25.301 25.245) (end 25.781 24.765) (width 0.1524) (layer F.Cu) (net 3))
 (segment (start 28.956 20.066) (end 29.65196 19.37004) (width 0.1524) (layer B.Cu) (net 3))
 (via (at 28.956 20.066) (size 0.6858) (drill 0.3302) (layers F.Cu B.Cu) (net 3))
 (segment (start 28.829 20.193) (end 28.956 20.066) (width 0.1524) (layer F.Cu) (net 3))
 (segment (start 28.829 24.257) (end 28.829 20.193) (width 0.1524) (layer F.Cu) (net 3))
 (segment (start 28.321 24.765) (end 28.829 24.257) (width 0.1524) (layer F.Cu) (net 3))
 (segment (start 25.781 24.765) (end 28.321 24.765) (width 0.1524) (layer F.Cu) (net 3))
 (segment (start 29.65196 19.37004) (end 29.65196 19.1668) (width 0.1524) (layer B.Cu) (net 3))
 (segment (start 25.60076 25.45424) (end 25.301 25.754) (width 0.25) (layer F.Cu) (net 3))
 (segment (start 27.6082 21.163) (end 27.6082 20.16158) (width 1) (layer B.Cu) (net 9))
 (segment (start 27.6082 20.16158) (end 27.65298 20.1168) (width 1) (layer B.Cu) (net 9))
 (segment (start 28.86202 23.3934) (end 28.86202 22.34758) (width 1) (layer B.Cu) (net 10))
 (segment (start 28.86202 22.34758) (end 28.8782 22.3314) (width 1) (layer B.Cu) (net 10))
 (segment (start 26.7589 23.8434) (end 26.7589 24.23926) (width 0.1524) (layer B.Cu) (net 4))
 (segment (start 26.7589 24.23926) (end 26.86304 24.3434) (width 0.1524) (layer B.Cu) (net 4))
 (segment (start 26.801 25.754) (end 26.801 24.40544) (width 0.1524) (layer B.Cu) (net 4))
 (segment (start 26.801 24.40544) (end 26.86304 24.3434) (width 0.1524) (layer B.Cu) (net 4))
 (segment (start 26.801 25.754) (end 26.801 25.299) (width 0.1524) (layer B.Cu) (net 4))
 (segment (start 31.0642 19.0406) (end 32.9852 19.0406) (width 1) (layer B.Cu) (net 6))
 (segment (start 32.9852 19.0406) (end 33.2994 19.3548) (width 1) (layer B.Cu) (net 6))
 (segment (start 34.2519 20.9202) (end 34.2519 20.3073) (width 1) (layer B.Cu) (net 6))
 (segment (start 34.2519 20.3073) (end 33.2994 19.3548) (width 1) (layer B.Cu) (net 6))
 (segment (start 33.401 20.971) (end 33.401 19.4564) (width 1) (layer B.Cu) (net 6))
 (segment (start 33.401 19.4564) (end 33.2994 19.3548) (width 1) (layer B.Cu) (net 6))
 (via (at 30.3055 25.6667) (size 0.6858) (drill 0.3302) (layers F.Cu B.Cu) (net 6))
 (segment (start 33.274 20.447) (end 34.163 20.447) (width 1) (layer B.Cu) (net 6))
 (via (at 34.163 20.447) (size 0.6858) (drill 0.3302) (layers F.Cu B.Cu) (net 6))
 (segment (start 33.528 21.082) (end 34.163 20.447) (width 1) (layer F.Cu) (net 6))
 (segment (start 33.528 25.654) (end 33.528 21.082) (width 1) (layer F.Cu) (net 6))
 (segment (start 33.655 25.781) (end 33.528 25.654) (width 1) (layer F.Cu) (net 6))
 (segment (start 30.4198 25.781) (end 33.655 25.781) (width 1) (layer F.Cu) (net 6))
 (segment (start 30.4198 25.781) (end 30.3055 25.6667) (width 1) (layer F.Cu) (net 6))
 (via (at 33.274 20.447) (size 0.6858) (drill 0.3302) (layers F.Cu B.Cu) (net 6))
 (segment (start 33.274 20.447) (end 33.655 20.828) (width 1) (layer F.Cu) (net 6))
 (segment (start 33.655 20.828) (end 33.655 20.955) (width 1) (layer F.Cu) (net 6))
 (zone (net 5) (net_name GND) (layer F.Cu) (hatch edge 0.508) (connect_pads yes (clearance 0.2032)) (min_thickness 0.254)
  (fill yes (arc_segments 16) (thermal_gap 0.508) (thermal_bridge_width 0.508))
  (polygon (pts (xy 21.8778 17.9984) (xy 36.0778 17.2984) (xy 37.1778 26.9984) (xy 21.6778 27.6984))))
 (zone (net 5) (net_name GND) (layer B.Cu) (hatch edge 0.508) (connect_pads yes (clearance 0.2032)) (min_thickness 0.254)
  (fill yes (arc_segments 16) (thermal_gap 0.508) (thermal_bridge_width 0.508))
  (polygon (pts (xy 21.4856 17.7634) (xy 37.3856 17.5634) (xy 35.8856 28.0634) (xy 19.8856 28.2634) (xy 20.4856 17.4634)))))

